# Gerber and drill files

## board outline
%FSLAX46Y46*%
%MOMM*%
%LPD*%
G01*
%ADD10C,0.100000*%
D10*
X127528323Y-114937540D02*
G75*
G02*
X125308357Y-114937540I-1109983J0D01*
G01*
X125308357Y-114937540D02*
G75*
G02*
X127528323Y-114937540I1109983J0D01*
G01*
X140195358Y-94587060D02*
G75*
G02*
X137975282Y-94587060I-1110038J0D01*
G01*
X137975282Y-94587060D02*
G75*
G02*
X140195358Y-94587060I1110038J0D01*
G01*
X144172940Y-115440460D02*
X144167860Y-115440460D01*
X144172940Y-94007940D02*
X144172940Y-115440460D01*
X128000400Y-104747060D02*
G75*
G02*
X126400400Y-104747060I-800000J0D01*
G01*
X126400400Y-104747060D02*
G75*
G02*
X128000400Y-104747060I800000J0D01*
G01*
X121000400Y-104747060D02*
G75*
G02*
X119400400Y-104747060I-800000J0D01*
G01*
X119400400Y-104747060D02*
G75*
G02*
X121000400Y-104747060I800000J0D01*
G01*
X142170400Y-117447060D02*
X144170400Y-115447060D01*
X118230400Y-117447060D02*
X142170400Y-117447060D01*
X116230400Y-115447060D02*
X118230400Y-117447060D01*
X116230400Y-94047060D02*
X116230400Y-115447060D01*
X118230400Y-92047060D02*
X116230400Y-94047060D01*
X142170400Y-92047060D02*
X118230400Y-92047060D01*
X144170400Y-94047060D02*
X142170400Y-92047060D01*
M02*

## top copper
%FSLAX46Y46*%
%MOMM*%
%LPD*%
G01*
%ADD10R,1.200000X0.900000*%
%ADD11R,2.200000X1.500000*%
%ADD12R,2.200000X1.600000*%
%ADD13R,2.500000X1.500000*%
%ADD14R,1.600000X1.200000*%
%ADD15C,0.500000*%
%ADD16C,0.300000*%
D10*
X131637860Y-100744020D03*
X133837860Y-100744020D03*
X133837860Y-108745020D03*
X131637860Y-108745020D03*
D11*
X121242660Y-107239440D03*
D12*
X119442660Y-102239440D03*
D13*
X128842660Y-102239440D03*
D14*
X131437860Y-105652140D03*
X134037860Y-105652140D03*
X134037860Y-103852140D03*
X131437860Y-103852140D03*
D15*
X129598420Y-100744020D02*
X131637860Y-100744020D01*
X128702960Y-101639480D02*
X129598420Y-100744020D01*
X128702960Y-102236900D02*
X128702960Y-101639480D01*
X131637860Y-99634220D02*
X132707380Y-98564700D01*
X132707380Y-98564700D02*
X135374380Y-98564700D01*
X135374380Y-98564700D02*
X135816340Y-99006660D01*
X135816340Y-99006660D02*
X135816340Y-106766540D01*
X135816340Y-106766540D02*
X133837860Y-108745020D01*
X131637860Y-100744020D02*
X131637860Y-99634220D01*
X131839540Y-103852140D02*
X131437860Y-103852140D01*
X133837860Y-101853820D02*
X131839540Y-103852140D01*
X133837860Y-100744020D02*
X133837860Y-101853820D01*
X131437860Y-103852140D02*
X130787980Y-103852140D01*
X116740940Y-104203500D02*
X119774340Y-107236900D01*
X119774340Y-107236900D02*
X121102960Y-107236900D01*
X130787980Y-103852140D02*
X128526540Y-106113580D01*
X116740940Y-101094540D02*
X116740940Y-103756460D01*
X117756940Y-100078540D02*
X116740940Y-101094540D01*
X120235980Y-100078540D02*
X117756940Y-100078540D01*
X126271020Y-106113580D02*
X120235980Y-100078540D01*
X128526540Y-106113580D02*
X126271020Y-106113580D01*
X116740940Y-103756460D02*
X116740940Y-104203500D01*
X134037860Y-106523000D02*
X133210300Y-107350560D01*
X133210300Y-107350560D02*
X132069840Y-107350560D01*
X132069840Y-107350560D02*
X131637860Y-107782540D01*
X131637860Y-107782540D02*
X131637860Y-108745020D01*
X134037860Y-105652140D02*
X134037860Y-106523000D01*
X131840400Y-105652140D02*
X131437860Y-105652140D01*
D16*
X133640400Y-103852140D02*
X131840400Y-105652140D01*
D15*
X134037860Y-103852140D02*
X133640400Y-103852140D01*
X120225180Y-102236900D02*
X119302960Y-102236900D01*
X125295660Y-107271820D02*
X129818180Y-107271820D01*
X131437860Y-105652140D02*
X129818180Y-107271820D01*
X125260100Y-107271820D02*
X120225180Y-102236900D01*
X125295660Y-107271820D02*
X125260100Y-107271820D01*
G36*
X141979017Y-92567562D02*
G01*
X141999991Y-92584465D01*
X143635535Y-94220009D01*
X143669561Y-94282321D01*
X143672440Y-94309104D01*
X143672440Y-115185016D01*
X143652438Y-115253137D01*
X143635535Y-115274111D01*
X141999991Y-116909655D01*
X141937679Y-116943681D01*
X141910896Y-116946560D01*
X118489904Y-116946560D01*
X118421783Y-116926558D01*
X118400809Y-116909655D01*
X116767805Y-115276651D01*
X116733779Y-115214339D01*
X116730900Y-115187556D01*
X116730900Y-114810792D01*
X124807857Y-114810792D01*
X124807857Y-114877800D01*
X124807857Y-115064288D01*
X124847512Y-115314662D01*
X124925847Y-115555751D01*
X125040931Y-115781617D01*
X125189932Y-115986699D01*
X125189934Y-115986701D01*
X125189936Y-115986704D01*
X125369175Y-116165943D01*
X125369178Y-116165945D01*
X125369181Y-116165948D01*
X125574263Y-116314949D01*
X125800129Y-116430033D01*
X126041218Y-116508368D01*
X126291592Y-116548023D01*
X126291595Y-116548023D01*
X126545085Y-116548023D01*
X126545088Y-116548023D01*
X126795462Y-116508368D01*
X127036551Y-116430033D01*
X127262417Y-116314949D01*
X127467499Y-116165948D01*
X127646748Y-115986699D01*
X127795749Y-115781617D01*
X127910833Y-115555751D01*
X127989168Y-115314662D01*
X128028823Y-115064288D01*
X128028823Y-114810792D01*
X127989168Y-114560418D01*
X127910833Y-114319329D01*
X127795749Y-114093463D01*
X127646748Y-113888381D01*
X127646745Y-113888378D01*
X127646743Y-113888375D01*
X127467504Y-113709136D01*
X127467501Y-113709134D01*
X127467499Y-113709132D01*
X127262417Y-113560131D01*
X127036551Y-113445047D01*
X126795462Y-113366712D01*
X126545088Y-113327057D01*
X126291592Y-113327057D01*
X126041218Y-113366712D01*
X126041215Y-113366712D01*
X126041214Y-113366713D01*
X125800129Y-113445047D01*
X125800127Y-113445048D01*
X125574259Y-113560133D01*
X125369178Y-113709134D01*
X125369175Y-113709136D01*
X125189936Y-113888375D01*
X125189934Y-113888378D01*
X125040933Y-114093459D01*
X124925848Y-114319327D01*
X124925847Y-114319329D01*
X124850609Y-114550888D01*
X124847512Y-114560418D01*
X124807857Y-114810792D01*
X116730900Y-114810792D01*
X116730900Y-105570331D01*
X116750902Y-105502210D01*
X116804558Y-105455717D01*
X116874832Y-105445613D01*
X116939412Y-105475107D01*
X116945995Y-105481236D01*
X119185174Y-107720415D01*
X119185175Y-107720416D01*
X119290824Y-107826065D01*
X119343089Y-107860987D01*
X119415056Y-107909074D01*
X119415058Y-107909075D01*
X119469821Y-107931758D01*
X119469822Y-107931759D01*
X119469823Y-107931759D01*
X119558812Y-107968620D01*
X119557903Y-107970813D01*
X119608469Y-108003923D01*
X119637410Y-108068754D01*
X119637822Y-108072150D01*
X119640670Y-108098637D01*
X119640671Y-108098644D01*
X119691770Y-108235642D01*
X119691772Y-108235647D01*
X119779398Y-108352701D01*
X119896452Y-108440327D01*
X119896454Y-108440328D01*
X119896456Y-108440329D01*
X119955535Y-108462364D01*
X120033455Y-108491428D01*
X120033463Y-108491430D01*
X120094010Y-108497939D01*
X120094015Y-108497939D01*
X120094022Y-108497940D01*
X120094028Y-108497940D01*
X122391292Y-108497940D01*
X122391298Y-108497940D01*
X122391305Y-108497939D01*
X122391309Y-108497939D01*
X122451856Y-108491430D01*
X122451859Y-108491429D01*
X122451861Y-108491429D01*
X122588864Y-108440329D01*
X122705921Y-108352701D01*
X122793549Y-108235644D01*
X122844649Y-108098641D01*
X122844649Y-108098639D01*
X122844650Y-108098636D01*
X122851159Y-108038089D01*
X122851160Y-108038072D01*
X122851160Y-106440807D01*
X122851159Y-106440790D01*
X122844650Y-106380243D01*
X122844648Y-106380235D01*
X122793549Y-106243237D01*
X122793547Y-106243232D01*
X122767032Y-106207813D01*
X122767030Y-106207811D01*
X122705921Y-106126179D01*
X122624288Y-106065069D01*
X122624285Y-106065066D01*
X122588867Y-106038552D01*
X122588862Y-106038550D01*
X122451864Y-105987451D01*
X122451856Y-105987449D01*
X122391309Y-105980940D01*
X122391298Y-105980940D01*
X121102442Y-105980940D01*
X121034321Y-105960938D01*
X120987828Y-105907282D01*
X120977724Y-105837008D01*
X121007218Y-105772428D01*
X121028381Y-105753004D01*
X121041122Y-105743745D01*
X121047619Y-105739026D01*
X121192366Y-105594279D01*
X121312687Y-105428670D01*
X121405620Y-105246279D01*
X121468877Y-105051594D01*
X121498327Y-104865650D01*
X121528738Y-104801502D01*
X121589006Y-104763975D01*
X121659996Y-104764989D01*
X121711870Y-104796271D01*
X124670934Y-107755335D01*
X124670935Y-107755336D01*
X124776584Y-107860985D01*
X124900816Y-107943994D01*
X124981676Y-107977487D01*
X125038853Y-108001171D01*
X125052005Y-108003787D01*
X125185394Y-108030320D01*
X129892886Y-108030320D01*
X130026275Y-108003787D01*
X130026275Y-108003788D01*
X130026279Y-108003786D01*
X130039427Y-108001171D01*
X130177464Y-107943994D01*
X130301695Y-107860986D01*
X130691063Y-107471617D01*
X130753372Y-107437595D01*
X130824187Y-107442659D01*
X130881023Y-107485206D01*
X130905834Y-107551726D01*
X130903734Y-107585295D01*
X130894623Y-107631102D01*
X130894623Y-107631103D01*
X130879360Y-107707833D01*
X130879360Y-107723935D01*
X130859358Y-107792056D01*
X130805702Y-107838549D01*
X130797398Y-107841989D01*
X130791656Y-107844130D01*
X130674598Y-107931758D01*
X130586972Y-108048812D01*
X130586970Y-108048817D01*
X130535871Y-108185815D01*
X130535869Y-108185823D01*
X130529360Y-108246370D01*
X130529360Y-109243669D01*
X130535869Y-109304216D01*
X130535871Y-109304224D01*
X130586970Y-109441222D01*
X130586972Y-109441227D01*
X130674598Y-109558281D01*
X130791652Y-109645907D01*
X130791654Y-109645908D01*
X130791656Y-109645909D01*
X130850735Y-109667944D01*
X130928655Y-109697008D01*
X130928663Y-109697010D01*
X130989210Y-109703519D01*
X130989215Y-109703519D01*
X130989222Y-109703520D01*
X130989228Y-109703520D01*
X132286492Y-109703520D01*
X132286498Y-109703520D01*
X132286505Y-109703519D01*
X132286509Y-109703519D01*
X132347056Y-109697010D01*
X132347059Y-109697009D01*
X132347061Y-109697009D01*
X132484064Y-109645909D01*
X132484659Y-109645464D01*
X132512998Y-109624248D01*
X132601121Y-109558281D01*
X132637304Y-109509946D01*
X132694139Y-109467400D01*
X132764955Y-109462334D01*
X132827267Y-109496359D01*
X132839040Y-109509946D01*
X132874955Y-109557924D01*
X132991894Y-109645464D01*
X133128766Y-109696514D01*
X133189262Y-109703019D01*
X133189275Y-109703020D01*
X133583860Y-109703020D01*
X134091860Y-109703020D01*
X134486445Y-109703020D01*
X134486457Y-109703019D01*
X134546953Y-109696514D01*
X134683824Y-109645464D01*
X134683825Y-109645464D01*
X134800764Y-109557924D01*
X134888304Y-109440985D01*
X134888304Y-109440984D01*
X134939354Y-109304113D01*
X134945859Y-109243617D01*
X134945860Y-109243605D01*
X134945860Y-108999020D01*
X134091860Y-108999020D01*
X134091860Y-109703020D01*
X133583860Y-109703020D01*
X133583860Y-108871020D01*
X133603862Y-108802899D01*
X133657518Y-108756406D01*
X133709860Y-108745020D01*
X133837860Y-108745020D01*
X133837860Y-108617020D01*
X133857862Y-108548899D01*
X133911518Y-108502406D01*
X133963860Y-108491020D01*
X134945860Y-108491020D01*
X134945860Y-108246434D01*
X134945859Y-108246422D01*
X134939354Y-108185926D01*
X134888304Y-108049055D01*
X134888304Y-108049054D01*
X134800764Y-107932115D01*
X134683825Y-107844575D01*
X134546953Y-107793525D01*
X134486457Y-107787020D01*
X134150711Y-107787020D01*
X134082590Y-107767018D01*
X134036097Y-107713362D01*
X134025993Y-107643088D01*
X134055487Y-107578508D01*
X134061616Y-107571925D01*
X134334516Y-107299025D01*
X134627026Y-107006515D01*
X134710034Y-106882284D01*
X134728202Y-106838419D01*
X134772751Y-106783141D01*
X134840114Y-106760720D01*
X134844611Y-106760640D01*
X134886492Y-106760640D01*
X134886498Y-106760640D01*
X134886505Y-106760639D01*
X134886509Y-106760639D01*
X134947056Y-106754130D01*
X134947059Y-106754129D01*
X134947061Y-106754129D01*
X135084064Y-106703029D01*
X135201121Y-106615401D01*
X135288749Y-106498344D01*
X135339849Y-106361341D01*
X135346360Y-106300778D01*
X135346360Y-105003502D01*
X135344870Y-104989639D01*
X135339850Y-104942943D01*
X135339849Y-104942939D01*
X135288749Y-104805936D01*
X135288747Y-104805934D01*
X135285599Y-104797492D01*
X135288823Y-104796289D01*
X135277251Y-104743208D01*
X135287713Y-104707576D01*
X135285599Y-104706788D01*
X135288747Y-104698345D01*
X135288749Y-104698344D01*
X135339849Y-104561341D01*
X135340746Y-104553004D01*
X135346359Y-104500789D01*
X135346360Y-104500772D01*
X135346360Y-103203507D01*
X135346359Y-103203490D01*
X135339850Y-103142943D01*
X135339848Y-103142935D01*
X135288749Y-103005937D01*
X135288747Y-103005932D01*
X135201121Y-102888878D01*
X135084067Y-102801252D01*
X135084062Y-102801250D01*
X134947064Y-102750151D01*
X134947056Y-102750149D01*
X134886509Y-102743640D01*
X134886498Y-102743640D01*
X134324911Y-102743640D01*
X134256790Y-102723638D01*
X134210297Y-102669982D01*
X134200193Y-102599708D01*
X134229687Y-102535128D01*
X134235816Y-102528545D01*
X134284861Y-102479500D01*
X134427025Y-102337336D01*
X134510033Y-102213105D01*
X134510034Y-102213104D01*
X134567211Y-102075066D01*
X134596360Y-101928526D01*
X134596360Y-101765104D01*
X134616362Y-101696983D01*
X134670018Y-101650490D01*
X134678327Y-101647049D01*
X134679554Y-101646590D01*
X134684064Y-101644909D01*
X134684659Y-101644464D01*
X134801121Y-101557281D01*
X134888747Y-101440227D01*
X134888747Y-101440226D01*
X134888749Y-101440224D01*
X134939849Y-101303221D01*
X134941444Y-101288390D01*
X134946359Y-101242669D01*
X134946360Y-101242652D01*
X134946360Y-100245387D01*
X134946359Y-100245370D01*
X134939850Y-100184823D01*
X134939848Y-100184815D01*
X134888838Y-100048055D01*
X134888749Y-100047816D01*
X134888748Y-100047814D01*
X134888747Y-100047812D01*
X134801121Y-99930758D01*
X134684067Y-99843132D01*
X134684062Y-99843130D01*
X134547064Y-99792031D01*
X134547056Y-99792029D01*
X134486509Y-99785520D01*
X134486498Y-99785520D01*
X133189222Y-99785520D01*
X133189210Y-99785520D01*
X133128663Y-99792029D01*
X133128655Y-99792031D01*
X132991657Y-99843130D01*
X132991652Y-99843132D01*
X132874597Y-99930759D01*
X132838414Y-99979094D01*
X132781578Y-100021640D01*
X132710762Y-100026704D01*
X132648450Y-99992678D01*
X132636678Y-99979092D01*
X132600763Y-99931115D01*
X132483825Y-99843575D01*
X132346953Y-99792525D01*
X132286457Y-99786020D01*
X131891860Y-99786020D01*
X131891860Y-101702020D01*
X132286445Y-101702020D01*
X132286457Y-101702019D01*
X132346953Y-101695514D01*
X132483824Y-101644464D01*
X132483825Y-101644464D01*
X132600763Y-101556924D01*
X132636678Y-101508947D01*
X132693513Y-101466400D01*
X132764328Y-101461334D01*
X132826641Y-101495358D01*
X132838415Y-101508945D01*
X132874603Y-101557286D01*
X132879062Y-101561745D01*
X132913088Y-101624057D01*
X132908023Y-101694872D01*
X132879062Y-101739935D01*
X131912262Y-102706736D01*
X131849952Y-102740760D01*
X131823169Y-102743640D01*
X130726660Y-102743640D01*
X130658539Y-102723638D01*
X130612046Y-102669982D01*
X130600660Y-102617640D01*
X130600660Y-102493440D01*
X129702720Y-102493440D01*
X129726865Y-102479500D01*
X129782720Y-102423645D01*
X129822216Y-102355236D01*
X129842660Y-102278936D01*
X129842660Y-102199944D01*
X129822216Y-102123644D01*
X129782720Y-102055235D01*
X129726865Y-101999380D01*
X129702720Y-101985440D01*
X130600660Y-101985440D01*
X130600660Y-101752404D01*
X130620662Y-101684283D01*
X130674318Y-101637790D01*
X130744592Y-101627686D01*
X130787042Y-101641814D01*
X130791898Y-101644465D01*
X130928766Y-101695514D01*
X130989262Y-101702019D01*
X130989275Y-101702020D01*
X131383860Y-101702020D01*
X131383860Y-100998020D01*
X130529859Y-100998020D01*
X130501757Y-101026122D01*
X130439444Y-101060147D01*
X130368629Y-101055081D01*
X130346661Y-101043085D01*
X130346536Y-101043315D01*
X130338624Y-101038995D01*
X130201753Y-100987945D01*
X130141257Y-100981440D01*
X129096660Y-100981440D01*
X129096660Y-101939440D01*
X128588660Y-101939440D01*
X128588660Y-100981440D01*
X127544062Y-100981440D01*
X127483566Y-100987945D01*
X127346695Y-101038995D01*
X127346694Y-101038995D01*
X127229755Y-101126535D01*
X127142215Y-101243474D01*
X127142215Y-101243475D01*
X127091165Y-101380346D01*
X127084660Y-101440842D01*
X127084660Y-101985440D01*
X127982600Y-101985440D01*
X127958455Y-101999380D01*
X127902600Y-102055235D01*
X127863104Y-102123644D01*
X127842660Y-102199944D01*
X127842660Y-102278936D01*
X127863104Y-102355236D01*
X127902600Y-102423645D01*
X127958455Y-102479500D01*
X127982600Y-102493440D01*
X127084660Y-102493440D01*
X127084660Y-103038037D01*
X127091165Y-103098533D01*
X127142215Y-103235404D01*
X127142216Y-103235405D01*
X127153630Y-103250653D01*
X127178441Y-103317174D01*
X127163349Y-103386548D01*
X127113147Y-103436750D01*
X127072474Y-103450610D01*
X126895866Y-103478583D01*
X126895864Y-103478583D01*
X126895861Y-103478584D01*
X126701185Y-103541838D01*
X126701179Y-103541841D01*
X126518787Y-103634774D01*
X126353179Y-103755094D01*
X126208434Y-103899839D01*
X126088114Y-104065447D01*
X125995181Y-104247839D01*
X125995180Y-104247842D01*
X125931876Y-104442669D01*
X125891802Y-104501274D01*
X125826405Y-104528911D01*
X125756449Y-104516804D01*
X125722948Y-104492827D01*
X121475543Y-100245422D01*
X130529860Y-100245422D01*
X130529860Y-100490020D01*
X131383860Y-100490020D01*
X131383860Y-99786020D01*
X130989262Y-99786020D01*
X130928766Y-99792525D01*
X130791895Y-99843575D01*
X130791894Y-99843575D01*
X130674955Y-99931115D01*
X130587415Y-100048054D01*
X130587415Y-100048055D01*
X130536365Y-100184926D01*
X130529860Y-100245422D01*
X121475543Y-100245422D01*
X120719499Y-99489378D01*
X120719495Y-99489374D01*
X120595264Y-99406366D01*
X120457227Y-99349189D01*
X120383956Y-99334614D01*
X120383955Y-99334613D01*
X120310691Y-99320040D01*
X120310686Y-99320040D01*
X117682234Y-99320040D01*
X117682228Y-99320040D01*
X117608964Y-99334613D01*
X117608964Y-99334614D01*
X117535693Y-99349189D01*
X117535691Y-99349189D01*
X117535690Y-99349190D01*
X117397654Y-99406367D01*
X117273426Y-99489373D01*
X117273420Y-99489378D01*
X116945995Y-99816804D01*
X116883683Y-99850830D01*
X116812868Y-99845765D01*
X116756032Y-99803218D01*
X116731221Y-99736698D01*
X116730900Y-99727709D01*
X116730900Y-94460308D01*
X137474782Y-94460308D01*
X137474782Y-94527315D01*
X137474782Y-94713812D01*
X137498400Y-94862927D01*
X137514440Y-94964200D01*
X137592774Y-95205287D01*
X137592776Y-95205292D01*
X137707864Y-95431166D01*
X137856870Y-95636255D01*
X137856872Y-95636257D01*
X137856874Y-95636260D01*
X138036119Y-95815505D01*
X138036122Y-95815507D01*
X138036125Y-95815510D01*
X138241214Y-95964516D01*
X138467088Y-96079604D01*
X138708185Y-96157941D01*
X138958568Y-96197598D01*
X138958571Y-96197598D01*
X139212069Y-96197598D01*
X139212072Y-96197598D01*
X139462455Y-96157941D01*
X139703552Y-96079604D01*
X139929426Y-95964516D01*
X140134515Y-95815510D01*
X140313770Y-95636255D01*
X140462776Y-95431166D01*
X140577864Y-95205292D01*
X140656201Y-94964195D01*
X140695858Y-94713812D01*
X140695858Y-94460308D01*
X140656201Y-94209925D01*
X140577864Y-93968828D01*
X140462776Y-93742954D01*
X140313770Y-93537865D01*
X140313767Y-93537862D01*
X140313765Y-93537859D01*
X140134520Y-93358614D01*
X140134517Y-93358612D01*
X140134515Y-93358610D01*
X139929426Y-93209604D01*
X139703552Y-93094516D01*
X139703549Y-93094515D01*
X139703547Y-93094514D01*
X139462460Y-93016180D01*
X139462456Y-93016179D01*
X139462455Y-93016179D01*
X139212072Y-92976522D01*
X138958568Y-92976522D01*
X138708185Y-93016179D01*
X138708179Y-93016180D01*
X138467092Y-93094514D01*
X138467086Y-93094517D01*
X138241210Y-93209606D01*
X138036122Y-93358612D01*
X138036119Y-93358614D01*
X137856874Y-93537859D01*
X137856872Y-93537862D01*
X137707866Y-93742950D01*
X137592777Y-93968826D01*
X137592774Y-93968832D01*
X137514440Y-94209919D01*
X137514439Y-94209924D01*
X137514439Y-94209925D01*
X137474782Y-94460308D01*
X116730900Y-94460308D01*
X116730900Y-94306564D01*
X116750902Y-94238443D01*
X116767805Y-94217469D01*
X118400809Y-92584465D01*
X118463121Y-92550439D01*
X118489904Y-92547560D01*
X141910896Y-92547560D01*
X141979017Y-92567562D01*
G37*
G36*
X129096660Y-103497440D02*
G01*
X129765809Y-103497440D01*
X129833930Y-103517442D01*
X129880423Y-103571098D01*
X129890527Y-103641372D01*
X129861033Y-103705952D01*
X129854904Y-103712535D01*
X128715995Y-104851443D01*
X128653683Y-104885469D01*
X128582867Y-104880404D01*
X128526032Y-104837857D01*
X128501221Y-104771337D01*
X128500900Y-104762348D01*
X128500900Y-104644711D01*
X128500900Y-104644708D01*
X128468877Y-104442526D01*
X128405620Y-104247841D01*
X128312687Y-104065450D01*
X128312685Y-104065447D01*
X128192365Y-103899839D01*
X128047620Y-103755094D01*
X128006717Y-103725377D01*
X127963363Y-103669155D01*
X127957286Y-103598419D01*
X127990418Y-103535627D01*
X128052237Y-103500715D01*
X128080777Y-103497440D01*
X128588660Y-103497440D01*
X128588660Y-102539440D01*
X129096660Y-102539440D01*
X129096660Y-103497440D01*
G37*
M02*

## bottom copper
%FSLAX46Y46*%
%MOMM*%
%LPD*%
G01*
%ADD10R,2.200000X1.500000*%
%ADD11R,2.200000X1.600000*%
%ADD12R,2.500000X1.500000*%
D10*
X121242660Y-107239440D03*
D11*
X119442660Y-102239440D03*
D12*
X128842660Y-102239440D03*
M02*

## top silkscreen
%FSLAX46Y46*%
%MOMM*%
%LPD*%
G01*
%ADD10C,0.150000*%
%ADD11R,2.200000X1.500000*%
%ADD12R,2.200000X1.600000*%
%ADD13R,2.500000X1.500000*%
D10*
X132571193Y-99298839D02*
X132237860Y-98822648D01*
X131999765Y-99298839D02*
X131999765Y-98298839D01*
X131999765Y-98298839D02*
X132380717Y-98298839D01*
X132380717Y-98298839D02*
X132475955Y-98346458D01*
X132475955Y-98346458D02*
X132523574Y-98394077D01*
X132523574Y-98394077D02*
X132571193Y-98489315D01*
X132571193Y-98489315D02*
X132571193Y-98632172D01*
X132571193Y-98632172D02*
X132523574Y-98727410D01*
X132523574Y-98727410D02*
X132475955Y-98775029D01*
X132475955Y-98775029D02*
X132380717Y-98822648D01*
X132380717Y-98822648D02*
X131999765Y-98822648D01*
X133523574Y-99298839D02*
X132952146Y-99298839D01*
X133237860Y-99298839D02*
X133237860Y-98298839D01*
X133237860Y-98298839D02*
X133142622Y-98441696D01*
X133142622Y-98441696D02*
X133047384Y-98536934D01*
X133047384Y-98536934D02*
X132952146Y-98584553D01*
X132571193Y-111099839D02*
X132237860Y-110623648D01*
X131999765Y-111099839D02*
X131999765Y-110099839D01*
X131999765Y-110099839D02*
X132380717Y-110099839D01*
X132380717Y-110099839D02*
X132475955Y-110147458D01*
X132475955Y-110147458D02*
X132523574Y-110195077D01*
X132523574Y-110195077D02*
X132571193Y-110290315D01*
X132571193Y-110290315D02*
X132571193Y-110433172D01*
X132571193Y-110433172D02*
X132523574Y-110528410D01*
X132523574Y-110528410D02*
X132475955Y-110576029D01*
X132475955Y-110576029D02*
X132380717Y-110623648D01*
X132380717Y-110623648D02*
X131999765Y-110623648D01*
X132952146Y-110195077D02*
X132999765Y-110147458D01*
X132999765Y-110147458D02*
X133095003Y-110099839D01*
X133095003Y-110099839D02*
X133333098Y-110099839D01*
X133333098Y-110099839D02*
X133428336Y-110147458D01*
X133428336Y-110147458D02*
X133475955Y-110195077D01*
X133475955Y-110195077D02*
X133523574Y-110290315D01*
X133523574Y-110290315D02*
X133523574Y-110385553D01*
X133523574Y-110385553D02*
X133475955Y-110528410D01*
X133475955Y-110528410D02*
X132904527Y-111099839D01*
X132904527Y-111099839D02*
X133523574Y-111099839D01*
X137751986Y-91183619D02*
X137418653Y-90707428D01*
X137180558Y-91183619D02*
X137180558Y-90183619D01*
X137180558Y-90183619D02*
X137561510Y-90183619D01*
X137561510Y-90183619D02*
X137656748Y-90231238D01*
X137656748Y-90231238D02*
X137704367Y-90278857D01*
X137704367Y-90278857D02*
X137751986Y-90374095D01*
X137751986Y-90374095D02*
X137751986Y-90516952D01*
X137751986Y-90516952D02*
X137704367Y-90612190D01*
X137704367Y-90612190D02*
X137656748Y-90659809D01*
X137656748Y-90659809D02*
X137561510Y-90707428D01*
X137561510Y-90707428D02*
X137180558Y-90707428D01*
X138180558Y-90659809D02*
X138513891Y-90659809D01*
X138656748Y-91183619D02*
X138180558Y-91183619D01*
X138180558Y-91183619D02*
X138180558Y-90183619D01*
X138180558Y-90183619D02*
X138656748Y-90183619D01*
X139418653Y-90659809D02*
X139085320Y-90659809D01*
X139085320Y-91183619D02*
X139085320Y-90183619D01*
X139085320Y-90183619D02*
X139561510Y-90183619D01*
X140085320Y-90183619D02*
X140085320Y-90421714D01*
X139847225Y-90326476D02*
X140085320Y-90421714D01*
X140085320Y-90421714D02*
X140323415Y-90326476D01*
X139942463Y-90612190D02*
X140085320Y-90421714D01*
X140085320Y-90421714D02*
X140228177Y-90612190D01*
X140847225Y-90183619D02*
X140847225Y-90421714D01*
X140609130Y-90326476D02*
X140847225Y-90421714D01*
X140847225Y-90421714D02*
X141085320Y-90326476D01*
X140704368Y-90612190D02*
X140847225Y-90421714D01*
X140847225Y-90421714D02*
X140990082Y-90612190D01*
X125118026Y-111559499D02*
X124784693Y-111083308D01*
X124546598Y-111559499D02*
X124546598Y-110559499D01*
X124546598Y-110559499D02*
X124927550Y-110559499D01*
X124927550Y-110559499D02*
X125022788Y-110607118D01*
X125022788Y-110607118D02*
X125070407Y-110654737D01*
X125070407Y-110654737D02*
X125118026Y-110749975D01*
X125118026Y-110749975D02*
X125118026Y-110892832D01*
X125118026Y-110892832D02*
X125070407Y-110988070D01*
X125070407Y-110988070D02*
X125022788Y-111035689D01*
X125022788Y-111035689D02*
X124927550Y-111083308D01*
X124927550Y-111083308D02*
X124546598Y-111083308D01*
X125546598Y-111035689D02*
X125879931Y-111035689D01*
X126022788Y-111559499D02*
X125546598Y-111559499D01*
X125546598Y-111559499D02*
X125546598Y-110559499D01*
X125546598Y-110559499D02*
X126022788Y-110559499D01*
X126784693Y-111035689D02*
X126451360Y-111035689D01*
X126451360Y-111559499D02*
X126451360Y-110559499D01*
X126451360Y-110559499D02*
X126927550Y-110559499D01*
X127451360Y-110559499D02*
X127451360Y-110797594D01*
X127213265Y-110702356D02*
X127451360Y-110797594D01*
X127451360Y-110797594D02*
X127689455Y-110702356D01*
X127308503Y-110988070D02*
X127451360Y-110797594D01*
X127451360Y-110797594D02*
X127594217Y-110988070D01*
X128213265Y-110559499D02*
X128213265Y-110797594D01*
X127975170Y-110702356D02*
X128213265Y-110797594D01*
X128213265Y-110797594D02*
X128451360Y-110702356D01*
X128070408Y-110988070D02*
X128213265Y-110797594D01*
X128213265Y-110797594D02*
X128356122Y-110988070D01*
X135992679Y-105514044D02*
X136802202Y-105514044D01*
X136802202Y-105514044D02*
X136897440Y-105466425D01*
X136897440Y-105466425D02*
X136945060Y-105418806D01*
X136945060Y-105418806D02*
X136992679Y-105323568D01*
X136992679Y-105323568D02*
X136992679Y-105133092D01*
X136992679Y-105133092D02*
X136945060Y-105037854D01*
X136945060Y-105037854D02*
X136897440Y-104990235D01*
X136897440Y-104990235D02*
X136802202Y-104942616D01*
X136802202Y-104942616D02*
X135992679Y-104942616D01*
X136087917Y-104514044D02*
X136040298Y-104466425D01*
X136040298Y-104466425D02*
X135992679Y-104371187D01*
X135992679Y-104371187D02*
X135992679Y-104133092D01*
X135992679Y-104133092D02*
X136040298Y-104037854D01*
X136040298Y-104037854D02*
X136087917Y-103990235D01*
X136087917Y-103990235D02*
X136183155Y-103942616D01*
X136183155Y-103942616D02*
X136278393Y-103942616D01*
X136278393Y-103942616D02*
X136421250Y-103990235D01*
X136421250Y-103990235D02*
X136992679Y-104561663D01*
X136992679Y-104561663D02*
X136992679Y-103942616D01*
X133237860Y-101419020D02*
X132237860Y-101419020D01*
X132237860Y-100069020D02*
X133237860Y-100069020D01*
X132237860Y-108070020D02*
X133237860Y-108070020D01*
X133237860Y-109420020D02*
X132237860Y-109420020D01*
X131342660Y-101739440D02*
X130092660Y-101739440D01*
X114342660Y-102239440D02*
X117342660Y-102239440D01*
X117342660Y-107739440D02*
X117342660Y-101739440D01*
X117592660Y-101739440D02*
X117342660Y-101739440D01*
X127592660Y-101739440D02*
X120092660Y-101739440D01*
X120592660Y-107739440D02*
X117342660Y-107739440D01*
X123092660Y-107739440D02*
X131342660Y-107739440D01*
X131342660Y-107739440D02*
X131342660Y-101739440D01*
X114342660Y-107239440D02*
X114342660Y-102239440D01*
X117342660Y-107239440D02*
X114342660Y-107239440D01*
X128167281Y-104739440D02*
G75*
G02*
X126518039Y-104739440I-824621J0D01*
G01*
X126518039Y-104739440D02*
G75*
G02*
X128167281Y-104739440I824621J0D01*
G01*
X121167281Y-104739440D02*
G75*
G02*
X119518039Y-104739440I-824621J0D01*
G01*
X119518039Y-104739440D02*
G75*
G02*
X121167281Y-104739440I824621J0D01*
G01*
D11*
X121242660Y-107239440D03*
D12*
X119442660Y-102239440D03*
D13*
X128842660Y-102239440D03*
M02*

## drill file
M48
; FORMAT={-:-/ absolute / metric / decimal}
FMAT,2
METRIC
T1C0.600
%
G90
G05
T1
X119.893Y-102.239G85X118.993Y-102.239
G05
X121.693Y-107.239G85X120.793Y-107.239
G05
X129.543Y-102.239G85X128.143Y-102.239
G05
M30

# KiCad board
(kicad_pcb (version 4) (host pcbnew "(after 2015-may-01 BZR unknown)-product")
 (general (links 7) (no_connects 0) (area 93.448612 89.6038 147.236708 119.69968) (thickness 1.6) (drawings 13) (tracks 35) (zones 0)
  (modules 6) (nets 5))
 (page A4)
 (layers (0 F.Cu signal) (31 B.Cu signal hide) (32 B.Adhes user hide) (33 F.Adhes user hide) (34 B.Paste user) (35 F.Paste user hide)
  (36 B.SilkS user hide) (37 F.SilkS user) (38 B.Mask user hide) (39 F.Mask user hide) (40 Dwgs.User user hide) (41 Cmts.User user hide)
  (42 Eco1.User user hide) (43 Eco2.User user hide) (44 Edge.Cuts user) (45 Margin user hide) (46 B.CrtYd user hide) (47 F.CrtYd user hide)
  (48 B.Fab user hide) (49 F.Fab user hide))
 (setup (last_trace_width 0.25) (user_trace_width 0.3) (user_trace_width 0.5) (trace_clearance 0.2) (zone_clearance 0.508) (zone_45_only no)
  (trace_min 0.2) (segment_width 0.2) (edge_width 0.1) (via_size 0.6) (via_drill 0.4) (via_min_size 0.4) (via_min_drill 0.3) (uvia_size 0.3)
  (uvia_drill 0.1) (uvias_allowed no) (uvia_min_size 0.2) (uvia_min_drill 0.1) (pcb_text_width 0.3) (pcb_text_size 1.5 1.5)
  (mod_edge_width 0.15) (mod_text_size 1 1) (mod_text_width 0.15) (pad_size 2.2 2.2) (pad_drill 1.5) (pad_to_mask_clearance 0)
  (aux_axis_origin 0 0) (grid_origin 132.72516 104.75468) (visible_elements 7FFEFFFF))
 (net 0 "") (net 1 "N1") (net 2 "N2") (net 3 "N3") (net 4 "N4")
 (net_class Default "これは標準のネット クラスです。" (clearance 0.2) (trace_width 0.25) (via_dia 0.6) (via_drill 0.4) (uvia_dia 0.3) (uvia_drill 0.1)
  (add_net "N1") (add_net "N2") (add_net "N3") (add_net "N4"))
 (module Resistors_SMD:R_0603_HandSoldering (layer F.Cu) (at 132.73786 100.74402)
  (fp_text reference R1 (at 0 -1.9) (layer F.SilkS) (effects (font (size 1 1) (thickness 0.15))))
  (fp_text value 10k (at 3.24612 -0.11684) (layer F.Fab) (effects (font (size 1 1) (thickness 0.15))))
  (fp_line (start 0.5 0.675) (end -0.5 0.675) (layer F.SilkS) (width 0.15))
  (fp_line (start -0.5 -0.675) (end 0.5 -0.675) (layer F.SilkS) (width 0.15))
  (pad 1 smd rect (at -1.1 0) (size 1.2 0.9) (layers F.Cu F.Paste F.Mask) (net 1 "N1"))
  (pad 2 smd rect (at 1.1 0) (size 1.2 0.9) (layers F.Cu F.Paste F.Mask) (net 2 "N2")))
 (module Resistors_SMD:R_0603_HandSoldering (layer F.Cu) (at 132.73786 108.74502 180)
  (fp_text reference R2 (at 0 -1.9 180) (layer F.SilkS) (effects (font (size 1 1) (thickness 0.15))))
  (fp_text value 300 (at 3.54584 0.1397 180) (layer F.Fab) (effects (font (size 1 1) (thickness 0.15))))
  (fp_line (start 0.5 0.675) (end -0.5 0.675) (layer F.SilkS) (width 0.15))
  (fp_line (start -0.5 -0.675) (end 0.5 -0.675) (layer F.SilkS) (width 0.15))
  (pad 1 smd rect (at -1.1 0 180) (size 1.2 0.9) (layers F.Cu F.Paste F.Mask) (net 1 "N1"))
  (pad 2 smd rect (at 1.1 0 180) (size 1.2 0.9) (layers F.Cu F.Paste F.Mask) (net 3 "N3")))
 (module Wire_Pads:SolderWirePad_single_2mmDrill (layer F.Cu) (at 139.08532 94.5388)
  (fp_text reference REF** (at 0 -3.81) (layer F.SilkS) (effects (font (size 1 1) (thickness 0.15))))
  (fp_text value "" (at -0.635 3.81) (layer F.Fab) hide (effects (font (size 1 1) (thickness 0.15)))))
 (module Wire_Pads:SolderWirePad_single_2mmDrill (layer F.Cu) (at 126.45136 114.91468)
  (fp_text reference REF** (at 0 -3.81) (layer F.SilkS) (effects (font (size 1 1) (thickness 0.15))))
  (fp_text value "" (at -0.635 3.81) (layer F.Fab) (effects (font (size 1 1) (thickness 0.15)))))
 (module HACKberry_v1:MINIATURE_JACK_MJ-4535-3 (layer F.Cu) (at 120.34266 104.73944 180)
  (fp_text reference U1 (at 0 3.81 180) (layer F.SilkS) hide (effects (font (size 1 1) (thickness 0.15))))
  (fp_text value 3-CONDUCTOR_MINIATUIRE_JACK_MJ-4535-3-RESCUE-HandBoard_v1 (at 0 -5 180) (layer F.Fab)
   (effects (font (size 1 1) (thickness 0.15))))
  (fp_line (start -11 3) (end -9.75 3) (layer F.SilkS) (width 0.15))
  (fp_line (start 6 2.5) (end 3 2.5) (layer F.SilkS) (width 0.15))
  (fp_line (start 3 -3) (end 3 3) (layer F.SilkS) (width 0.15))
  (fp_line (start 2.75 3) (end 3 3) (layer F.SilkS) (width 0.15))
  (fp_line (start -7.25 3) (end 0.25 3) (layer F.SilkS) (width 0.15))
  (fp_line (start -0.25 -3) (end 3 -3) (layer F.SilkS) (width 0.15))
  (fp_line (start -2.75 -3) (end -11 -3) (layer F.SilkS) (width 0.15))
  (fp_line (start -11 -3) (end -11 3) (layer F.SilkS) (width 0.15))
  (fp_line (start 6 -2.5) (end 6 2.5) (layer F.SilkS) (width 0.15))
  (fp_line (start 3 -2.5) (end 6 -2.5) (layer F.SilkS) (width 0.15))
  (fp_circle (center -7 0) (end -6.8 0.8) (layer F.SilkS) (width 0.15))
  (fp_circle (center 0 0) (end -0.2 0.8) (layer F.SilkS) (width 0.15))
  (pad 4 thru_hole rect (at -0.9 -2.5 180) (size 2.2 1.5) (drill oval 1.5 0.6) (layers *.Cu *.Mask F.SilkS) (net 2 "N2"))
  (pad 2 thru_hole rect (at 0.9 2.5 180) (size 2.2 1.6) (drill oval 1.5 0.6) (layers *.Cu *.Mask F.SilkS) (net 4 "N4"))
  (pad 1 thru_hole rect (at -8.5 2.5 180) (size 2.5 1.5) (drill oval 2 0.6) (layers *.Cu *.Mask F.SilkS) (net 1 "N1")))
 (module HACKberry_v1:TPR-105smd (layer F.Cu) (at 132.73786 104.75214 90)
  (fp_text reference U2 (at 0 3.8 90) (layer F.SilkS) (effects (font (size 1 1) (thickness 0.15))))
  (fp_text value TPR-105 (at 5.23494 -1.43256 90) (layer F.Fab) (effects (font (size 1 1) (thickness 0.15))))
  (pad 1 smd rect (at -0.9 -1.3 90) (size 1.2 1.6) (layers F.Cu F.Paste F.Mask) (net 4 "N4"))
  (pad 2 smd rect (at -0.9 1.3 90) (size 1.2 1.6) (layers F.Cu F.Paste F.Mask) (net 3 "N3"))
  (pad 3 smd rect (at 0.9 1.3 90) (size 1.2 1.6) (layers F.Cu F.Paste F.Mask) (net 4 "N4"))
  (pad 4 smd rect (at 0.9 -1.3 90) (size 1.2 1.6) (layers F.Cu F.Paste F.Mask) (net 2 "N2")))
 (gr_circle (center 126.41834 114.93754) (end 126.42088 113.82756) (layer Edge.Cuts) (width 0.1))
 (gr_circle (center 139.08532 94.58706) (end 139.192 93.48216) (layer Edge.Cuts) (width 0.1))
 (gr_line (start 144.17294 115.44046) (end 144.16786 115.44046) (angle 90) (layer Edge.Cuts) (width 0.1))
 (gr_line (start 144.17294 94.00794) (end 144.17294 115.44046) (angle 90) (layer Edge.Cuts) (width 0.1))
 (gr_circle (center 127.2004 104.74706) (end 127.2004 105.54706) (layer Edge.Cuts) (width 0.1))
 (gr_circle (center 120.2004 104.74706) (end 120.2004 105.54706) (layer Edge.Cuts) (width 0.1))
 (gr_line (start 142.1704 117.44706) (end 144.1704 115.44706) (layer Edge.Cuts) (width 0.1))
 (gr_line (start 118.2304 117.44706) (end 142.1704 117.44706) (layer Edge.Cuts) (width 0.1))
 (gr_line (start 116.2304 115.44706) (end 118.2304 117.44706) (layer Edge.Cuts) (width 0.1))
 (gr_line (start 116.2304 94.04706) (end 116.2304 115.44706) (layer Edge.Cuts) (width 0.1))
 (gr_line (start 118.2304 92.04706) (end 116.2304 94.04706) (layer Edge.Cuts) (width 0.1))
 (gr_line (start 142.1704 92.04706) (end 118.2304 92.04706) (layer Edge.Cuts) (width 0.1))
 (gr_line (start 144.1704 94.04706) (end 142.1704 92.04706) (layer Edge.Cuts) (width 0.1))
 (segment (start 129.59842 100.74402) (end 131.63786 100.74402) (width 0.5) (layer F.Cu) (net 1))
 (segment (start 128.70296 101.63948) (end 129.59842 100.74402) (width 0.5) (layer F.Cu) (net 1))
 (segment (start 128.70296 102.2369) (end 128.70296 101.63948) (width 0.5) (layer F.Cu) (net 1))
 (segment (start 131.63786 99.63422) (end 132.70738 98.5647) (width 0.5) (layer F.Cu) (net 1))
 (segment (start 132.70738 98.5647) (end 135.37438 98.5647) (width 0.5) (layer F.Cu) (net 1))
 (segment (start 135.37438 98.5647) (end 135.81634 99.00666) (width 0.5) (layer F.Cu) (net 1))
 (segment (start 135.81634 99.00666) (end 135.81634 106.76654) (width 0.5) (layer F.Cu) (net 1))
 (segment (start 135.81634 106.76654) (end 133.83786 108.74502) (width 0.5) (layer F.Cu) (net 1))
 (segment (start 131.63786 100.74402) (end 131.63786 99.63422) (width 0.5) (layer F.Cu) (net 1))
 (segment (start 131.83954 103.85214) (end 131.43786 103.85214) (width 0.5) (layer F.Cu) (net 2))
 (segment (start 133.83786 101.85382) (end 131.83954 103.85214) (width 0.5) (layer F.Cu) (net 2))
 (segment (start 133.83786 100.74402) (end 133.83786 101.85382) (width 0.5) (layer F.Cu) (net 2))
 (segment (start 131.43786 103.85214) (end 130.78798 103.85214) (width 0.5) (layer F.Cu) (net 2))
 (segment (start 116.74094 104.2035) (end 119.77434 107.2369) (width 0.5) (layer F.Cu) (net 2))
 (segment (start 119.77434 107.2369) (end 121.10296 107.2369) (width 0.5) (layer F.Cu) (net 2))
 (segment (start 130.78798 103.85214) (end 128.52654 106.11358) (width 0.5) (layer F.Cu) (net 2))
 (segment (start 116.74094 101.09454) (end 116.74094 103.75646) (width 0.5) (layer F.Cu) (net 2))
 (segment (start 117.75694 100.07854) (end 116.74094 101.09454) (width 0.5) (layer F.Cu) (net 2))
 (segment (start 120.23598 100.07854) (end 117.75694 100.07854) (width 0.5) (layer F.Cu) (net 2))
 (segment (start 126.27102 106.11358) (end 120.23598 100.07854) (width 0.5) (layer F.Cu) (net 2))
 (segment (start 128.52654 106.11358) (end 126.27102 106.11358) (width 0.5) (layer F.Cu) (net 2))
 (segment (start 116.74094 103.75646) (end 116.74094 104.2035) (width 0.5) (layer F.Cu) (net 2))
 (segment (start 134.03786 106.523) (end 133.2103 107.35056) (width 0.5) (layer F.Cu) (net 3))
 (segment (start 133.2103 107.35056) (end 132.06984 107.35056) (width 0.5) (layer F.Cu) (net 3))
 (segment (start 132.06984 107.35056) (end 131.63786 107.78254) (width 0.5) (layer F.Cu) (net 3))
 (segment (start 131.63786 107.78254) (end 131.63786 108.74502) (width 0.5) (layer F.Cu) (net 3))
 (segment (start 134.03786 105.65214) (end 134.03786 106.523) (width 0.5) (layer F.Cu) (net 3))
 (segment (start 131.8404 105.65214) (end 131.43786 105.65214) (width 0.5) (layer F.Cu) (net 4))
 (segment (start 133.6404 103.85214) (end 131.8404 105.65214) (width 0.3) (layer F.Cu) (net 4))
 (segment (start 134.03786 103.85214) (end 133.6404 103.85214) (width 0.5) (layer F.Cu) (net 4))
 (segment (start 120.22518 102.2369) (end 119.30296 102.2369) (width 0.5) (layer F.Cu) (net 4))
 (segment (start 125.29566 107.27182) (end 129.81818 107.27182) (width 0.5) (layer F.Cu) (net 4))
 (segment (start 131.43786 105.65214) (end 129.81818 107.27182) (width 0.5) (layer F.Cu) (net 4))
 (segment (start 125.2601 107.27182) (end 120.22518 102.2369) (width 0.5) (layer F.Cu) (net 4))
 (segment (start 125.29566 107.27182) (end 125.2601 107.27182) (width 0.5) (layer F.Cu) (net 4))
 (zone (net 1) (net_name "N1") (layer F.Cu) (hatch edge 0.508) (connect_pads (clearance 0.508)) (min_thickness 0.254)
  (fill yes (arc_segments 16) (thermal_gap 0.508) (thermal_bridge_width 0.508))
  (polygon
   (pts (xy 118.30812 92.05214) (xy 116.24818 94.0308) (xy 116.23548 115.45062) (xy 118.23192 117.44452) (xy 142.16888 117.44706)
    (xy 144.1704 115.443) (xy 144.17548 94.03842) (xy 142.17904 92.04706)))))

